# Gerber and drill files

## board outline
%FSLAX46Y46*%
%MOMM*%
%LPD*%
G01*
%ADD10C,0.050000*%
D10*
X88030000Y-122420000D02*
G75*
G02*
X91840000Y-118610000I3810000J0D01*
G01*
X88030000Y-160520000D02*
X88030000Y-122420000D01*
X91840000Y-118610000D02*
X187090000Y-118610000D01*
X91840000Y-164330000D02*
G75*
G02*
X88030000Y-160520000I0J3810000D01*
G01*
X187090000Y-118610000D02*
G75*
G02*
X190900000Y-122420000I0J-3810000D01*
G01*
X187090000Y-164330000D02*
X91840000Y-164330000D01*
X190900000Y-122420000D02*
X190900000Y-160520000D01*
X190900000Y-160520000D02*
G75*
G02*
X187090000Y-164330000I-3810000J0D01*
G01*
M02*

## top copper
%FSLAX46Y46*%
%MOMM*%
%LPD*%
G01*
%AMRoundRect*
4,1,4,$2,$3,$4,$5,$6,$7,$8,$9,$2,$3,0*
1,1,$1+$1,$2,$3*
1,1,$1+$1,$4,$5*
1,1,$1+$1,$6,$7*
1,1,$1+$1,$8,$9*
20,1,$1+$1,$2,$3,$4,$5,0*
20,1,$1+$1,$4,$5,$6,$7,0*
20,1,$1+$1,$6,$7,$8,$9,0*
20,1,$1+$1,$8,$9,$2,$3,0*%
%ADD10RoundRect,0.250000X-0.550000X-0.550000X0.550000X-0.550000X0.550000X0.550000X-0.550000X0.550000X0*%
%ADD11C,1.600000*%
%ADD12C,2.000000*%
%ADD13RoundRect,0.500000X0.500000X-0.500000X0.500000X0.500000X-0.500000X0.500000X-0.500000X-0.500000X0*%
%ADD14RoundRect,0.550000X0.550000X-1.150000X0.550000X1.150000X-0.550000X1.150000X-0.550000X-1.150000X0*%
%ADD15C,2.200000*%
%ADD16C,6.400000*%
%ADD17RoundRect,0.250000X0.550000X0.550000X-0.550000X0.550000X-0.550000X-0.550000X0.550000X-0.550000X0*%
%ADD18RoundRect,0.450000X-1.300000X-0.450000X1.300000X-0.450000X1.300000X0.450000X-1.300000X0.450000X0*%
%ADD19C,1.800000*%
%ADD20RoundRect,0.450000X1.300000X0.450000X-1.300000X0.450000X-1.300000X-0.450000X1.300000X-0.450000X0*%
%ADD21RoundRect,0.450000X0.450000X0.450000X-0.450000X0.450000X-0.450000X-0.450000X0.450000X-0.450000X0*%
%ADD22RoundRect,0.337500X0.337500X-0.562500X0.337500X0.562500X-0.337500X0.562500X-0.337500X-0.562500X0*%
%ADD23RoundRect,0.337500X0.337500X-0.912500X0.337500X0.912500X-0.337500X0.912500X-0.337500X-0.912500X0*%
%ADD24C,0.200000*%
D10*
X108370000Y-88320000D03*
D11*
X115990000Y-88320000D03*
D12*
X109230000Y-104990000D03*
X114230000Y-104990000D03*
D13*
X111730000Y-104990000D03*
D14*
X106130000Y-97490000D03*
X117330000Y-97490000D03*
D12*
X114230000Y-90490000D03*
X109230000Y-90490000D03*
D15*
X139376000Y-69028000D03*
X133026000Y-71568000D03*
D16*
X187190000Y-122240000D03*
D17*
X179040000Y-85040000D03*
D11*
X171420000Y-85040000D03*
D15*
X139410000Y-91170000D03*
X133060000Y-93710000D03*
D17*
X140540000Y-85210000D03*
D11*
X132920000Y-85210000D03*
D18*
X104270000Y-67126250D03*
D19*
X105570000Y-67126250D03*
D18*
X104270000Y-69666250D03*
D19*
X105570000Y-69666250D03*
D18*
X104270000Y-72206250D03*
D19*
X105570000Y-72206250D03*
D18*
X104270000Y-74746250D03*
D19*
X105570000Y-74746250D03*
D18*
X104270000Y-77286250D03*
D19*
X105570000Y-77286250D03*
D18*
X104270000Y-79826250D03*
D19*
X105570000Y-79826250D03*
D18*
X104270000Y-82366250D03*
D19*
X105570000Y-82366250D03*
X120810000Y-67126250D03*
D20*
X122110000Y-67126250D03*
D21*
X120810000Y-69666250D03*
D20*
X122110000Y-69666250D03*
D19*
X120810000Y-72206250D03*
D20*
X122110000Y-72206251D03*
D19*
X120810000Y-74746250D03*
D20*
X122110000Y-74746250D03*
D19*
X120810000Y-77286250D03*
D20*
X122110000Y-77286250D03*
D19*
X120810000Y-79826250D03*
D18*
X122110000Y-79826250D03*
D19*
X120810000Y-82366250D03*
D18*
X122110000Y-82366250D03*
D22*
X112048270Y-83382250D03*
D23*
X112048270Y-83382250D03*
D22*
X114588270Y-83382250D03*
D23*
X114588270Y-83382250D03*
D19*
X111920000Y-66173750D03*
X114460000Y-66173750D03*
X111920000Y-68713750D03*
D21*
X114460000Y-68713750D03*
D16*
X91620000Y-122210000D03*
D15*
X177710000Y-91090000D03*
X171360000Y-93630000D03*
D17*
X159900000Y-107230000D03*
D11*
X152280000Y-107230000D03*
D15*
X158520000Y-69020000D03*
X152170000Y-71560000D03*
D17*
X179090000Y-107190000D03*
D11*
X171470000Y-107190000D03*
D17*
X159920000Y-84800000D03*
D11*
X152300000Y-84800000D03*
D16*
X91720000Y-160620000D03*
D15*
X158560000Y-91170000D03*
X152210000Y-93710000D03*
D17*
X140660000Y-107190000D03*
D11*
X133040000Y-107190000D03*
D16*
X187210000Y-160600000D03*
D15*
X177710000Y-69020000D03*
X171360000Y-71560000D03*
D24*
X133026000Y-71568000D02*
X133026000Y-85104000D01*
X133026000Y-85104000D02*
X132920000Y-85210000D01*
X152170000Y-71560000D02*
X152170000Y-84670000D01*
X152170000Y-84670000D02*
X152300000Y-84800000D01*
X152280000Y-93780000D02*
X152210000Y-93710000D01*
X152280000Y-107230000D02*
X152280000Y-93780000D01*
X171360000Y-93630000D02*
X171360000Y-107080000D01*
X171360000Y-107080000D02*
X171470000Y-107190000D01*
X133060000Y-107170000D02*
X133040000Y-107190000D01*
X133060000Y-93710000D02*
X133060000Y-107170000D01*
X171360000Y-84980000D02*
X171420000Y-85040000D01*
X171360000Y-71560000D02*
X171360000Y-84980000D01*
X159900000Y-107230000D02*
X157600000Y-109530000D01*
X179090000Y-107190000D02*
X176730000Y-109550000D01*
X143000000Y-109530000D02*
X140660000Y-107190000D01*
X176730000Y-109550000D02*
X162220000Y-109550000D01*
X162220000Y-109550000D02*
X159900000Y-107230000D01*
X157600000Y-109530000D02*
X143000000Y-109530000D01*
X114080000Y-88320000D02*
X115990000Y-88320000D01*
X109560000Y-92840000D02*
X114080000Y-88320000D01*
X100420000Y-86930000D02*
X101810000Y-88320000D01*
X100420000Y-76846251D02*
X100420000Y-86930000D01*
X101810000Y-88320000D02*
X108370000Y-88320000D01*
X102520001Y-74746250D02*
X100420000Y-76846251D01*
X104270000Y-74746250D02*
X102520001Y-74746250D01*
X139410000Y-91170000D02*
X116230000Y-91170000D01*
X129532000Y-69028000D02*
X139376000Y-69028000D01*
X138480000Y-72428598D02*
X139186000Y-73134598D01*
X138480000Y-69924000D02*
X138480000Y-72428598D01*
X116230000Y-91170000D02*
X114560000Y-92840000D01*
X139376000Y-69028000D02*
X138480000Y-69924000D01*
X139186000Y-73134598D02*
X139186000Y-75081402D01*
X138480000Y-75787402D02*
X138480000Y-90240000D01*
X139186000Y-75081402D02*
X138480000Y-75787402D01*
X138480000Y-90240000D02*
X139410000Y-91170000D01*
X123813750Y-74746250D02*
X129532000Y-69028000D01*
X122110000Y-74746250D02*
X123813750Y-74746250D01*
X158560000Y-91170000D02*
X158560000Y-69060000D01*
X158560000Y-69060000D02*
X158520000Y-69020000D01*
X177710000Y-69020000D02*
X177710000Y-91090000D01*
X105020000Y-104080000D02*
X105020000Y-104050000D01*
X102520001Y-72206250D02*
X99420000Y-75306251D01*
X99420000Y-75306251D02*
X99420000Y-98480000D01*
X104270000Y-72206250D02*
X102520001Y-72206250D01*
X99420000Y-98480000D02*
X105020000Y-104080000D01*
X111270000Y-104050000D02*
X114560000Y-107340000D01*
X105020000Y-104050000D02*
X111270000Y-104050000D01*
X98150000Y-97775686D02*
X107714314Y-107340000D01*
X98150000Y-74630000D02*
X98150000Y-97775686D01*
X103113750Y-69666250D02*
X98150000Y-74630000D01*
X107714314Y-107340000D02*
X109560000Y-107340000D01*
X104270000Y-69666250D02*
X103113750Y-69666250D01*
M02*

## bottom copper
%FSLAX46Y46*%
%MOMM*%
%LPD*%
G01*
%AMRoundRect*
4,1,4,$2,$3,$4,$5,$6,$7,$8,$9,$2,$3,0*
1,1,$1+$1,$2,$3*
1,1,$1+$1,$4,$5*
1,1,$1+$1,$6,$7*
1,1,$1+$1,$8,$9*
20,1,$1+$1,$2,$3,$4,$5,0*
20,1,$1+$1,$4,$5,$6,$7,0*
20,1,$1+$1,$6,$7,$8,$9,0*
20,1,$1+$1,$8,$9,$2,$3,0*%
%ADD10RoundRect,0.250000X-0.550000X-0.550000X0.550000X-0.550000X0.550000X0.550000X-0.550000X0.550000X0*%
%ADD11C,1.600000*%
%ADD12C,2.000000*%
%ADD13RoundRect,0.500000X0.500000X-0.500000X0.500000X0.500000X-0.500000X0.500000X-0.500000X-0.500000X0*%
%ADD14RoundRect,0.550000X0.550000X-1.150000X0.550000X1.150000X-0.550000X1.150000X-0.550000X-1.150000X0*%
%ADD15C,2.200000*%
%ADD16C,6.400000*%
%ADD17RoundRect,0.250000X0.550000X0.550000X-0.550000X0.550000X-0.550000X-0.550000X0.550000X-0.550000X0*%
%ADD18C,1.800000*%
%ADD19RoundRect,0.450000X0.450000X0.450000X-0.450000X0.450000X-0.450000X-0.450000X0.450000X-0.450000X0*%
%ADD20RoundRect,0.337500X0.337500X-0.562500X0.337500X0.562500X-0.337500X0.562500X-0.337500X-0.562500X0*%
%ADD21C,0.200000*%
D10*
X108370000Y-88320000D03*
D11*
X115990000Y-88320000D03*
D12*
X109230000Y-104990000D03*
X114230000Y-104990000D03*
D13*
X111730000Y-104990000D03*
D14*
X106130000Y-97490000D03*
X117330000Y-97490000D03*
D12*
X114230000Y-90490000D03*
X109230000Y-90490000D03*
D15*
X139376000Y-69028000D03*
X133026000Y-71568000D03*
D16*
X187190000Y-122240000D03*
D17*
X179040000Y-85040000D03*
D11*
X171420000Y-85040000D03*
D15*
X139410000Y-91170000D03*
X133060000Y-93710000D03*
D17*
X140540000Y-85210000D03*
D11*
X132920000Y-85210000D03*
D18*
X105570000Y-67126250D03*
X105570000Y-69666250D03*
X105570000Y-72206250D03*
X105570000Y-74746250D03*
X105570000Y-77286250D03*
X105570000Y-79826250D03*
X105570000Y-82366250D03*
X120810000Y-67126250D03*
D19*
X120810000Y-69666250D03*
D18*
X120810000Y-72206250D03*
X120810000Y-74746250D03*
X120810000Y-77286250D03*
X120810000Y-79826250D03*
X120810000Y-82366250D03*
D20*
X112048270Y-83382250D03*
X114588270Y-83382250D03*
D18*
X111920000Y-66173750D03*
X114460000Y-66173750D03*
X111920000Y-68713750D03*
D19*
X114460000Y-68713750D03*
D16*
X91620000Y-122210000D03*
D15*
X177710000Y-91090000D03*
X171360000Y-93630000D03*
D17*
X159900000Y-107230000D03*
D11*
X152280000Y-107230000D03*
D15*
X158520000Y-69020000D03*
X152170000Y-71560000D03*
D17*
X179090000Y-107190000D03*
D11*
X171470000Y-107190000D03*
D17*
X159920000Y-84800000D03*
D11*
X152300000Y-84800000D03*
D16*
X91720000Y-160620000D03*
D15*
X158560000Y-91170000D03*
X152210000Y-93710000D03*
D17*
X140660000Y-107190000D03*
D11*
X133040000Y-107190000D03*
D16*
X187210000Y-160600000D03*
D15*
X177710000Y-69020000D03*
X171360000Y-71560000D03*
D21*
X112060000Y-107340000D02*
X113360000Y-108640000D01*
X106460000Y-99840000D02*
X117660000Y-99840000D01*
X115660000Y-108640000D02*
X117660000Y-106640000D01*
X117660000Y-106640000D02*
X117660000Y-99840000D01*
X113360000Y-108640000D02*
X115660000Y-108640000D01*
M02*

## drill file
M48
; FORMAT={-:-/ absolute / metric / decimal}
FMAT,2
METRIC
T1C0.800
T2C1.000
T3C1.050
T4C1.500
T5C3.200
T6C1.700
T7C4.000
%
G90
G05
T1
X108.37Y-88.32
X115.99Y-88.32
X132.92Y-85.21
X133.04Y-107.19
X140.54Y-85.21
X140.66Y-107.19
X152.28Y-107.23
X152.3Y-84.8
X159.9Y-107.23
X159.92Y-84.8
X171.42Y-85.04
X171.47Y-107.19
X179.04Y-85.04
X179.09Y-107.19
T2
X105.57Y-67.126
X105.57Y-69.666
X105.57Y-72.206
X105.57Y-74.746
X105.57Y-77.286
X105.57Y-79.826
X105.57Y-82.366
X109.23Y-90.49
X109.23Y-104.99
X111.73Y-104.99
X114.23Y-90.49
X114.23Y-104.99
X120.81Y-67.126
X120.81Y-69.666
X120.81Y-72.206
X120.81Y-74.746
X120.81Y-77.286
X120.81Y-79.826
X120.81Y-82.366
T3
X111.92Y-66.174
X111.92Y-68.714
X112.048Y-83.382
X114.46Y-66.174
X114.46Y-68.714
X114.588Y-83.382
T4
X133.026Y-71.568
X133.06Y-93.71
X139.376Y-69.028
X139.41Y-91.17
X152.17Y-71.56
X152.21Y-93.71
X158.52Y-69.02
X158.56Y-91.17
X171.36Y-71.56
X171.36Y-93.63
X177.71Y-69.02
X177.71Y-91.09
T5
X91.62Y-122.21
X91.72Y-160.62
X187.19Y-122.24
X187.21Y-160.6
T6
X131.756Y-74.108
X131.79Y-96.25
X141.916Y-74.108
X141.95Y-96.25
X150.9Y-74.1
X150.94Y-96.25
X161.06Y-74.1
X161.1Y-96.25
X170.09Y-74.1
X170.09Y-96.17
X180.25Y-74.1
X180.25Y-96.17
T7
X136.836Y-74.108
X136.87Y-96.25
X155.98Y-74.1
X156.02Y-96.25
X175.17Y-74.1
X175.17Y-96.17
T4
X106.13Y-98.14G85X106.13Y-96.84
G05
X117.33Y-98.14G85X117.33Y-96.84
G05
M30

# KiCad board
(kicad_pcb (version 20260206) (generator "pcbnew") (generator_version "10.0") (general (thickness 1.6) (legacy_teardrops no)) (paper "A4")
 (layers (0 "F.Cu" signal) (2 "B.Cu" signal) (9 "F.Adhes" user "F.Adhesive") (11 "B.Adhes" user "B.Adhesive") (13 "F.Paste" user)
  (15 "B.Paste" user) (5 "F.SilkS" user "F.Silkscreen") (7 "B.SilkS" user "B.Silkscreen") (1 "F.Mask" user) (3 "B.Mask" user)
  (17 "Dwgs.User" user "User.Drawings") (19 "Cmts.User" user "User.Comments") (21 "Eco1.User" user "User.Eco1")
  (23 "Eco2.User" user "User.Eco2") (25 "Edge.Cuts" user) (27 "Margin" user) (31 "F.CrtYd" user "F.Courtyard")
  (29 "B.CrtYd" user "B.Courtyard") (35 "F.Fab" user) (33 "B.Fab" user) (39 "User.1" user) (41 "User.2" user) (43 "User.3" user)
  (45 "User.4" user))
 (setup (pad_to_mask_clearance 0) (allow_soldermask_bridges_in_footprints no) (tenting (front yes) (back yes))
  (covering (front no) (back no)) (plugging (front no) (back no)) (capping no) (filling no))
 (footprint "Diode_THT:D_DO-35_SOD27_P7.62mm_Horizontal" (layer "F.Cu") (at 108.37 88.32)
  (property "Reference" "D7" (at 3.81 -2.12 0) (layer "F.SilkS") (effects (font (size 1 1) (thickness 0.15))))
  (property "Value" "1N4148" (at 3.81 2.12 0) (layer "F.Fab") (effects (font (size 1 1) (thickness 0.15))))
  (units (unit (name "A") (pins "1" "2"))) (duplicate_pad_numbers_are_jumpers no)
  (pad "1" thru_hole roundrect (at 0 0) (size 1.6 1.6) (drill 0.8) (layers "*.Cu" "*.Mask") (remove_unused_layers no)
   (roundrect_rratio 0.15625) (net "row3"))
  (pad "2" thru_hole circle (at 7.62 0) (size 1.6 1.6) (drill 0.8) (layers "*.Cu" "*.Mask") (remove_unused_layers no) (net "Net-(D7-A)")))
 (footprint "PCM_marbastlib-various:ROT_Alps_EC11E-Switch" (layer "F.Cu") (at 111.73 97.49)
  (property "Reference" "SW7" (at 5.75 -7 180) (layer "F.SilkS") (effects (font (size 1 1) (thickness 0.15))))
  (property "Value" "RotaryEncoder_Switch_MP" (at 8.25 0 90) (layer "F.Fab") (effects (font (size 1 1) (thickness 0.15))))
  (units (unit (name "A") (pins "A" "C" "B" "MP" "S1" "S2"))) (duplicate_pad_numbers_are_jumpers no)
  (pad "A" thru_hole circle (at -2.5 7.5 90) (size 2 2) (drill 1) (layers "*.Cu" "B.Mask") (remove_unused_layers no) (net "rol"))
  (pad "B" thru_hole circle (at 2.5 7.5 90) (size 2 2) (drill 1) (layers "*.Cu" "B.Mask") (remove_unused_layers no) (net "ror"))
  (pad "C" thru_hole roundrect (at 0 7.5 90) (size 2 2) (drill 1) (layers "*.Cu" "B.Mask") (remove_unused_layers no) (roundrect_rratio 0.25)
   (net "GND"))
  (pad "MP" thru_hole roundrect (at -5.6 0 90) (size 3.4 2.2) (drill oval 2.8 1.5) (layers "*.Cu" "B.Mask") (remove_unused_layers no)
   (roundrect_rratio 0.25) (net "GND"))
  (pad "MP" thru_hole roundrect (at 5.6 0 90) (size 3.4 2.2) (drill oval 2.8 1.5) (layers "*.Cu" "B.Mask") (remove_unused_layers no)
   (roundrect_rratio 0.25) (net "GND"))
  (pad "S1" thru_hole circle (at 2.5 -7 90) (size 2 2) (drill 1) (layers "*.Cu" "B.Mask") (remove_unused_layers no) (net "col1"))
  (pad "S2" thru_hole circle (at -2.5 -7 90) (size 2 2) (drill 1) (layers "*.Cu" "B.Mask") (remove_unused_layers no) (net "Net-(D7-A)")))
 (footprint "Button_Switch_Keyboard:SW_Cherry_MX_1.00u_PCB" (layer "F.Cu") (at 139.376 69.028)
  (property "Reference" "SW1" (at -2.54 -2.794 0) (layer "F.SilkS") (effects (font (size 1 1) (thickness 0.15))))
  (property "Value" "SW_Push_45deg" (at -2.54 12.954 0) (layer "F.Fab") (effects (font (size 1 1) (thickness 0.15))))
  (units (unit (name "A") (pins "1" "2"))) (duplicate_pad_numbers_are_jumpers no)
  (pad "" np_thru_hole circle (at -7.62 5.08) (size 1.7 1.7) (drill 1.7) (layers "*.Cu" "*.Mask"))
  (pad "" np_thru_hole circle (at -2.54 5.08) (size 4 4) (drill 4) (layers "*.Cu" "*.Mask"))
  (pad "" np_thru_hole circle (at 2.54 5.08) (size 1.7 1.7) (drill 1.7) (layers "*.Cu" "*.Mask"))
  (pad "1" thru_hole circle (at 0 0) (size 2.2 2.2) (drill 1.5) (layers "*.Cu" "*.Mask") (remove_unused_layers no) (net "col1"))
  (pad "2" thru_hole circle (at -6.35 2.54) (size 2.2 2.2) (drill 1.5) (layers "*.Cu" "*.Mask") (remove_unused_layers no) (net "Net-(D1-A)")))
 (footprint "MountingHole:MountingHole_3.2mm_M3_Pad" (layer "F.Cu") (at 187.19 122.24)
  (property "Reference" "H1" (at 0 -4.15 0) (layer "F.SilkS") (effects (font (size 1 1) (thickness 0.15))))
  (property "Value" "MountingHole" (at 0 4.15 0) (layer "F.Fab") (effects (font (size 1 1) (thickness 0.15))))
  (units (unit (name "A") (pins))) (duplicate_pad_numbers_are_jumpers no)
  (pad "1" thru_hole circle (at 0 0) (size 6.4 6.4) (drill 3.2) (layers "*.Cu" "*.Mask") (remove_unused_layers no) (zone_connect 2)))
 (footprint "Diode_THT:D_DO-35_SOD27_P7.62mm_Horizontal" (layer "F.Cu") (at 179.04 85.04 180)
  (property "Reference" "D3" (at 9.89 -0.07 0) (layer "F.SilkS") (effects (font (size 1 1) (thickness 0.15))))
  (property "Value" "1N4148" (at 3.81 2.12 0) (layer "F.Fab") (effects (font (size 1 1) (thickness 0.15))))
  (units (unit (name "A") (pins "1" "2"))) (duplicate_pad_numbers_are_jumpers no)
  (pad "1" thru_hole roundrect (at 0 0 180) (size 1.6 1.6) (drill 0.8) (layers "*.Cu" "*.Mask") (remove_unused_layers no)
   (roundrect_rratio 0.15625) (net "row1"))
  (pad "2" thru_hole circle (at 7.62 0 180) (size 1.6 1.6) (drill 0.8) (layers "*.Cu" "*.Mask") (remove_unused_layers no) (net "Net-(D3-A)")))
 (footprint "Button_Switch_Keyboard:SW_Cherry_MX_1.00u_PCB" (layer "F.Cu") (at 139.41 91.17)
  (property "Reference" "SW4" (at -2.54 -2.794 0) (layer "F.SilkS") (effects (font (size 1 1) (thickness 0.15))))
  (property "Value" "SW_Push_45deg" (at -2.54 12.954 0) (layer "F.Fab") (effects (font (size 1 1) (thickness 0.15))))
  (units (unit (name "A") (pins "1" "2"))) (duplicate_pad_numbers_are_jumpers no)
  (pad "" np_thru_hole circle (at -7.62 5.08) (size 1.7 1.7) (drill 1.7) (layers "*.Cu" "*.Mask"))
  (pad "" np_thru_hole circle (at -2.54 5.08) (size 4 4) (drill 4) (layers "*.Cu" "*.Mask"))
  (pad "" np_thru_hole circle (at 2.54 5.08) (size 1.7 1.7) (drill 1.7) (layers "*.Cu" "*.Mask"))
  (pad "1" thru_hole circle (at 0 0) (size 2.2 2.2) (drill 1.5) (layers "*.Cu" "*.Mask") (remove_unused_layers no) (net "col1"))
  (pad "2" thru_hole circle (at -6.35 2.54) (size 2.2 2.2) (drill 1.5) (layers "*.Cu" "*.Mask") (remove_unused_layers no) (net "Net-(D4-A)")))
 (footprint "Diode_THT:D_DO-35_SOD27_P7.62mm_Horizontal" (layer "F.Cu") (at 140.54 85.21 180)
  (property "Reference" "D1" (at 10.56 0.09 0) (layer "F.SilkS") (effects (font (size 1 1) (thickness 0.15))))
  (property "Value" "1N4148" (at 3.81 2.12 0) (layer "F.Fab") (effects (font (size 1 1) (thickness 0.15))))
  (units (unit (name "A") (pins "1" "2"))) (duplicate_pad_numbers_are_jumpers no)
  (pad "1" thru_hole roundrect (at 0 0 180) (size 1.6 1.6) (drill 0.8) (layers "*.Cu" "*.Mask") (remove_unused_layers no)
   (roundrect_rratio 0.15625) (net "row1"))
  (pad "2" thru_hole circle (at 7.62 0 180) (size 1.6 1.6) (drill 0.8) (layers "*.Cu" "*.Mask") (remove_unused_layers no) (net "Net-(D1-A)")))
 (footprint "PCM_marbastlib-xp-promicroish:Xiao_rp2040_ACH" (layer "F.Cu") (at 113.19 74.74625)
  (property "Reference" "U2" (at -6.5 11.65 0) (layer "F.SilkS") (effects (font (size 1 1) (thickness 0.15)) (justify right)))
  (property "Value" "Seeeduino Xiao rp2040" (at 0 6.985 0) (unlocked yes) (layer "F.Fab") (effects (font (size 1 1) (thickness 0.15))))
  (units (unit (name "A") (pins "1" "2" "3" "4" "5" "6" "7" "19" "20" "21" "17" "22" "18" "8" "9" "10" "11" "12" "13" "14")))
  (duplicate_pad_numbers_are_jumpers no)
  (pad "1" smd roundrect (at -8.92 -7.62) (size 3.5 1.8) (layers "F.Cu" "F.Mask") (roundrect_rratio 0.25) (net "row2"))
  (pad "1" thru_hole circle (at -7.62 -7.62) (size 1.8 1.8) (drill 1) (layers "*.Cu" "*.Mask") (remove_unused_layers no) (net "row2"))
  (pad "2" smd roundrect (at -8.92 -5.08) (size 3.5 1.8) (layers "F.Cu" "F.Mask") (roundrect_rratio 0.25) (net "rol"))
  (pad "2" thru_hole circle (at -7.62 -5.08) (size 1.8 1.8) (drill 1) (layers "*.Cu" "*.Mask") (remove_unused_layers no) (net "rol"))
  (pad "3" smd roundrect (at -8.92 -2.54) (size 3.5 1.8) (layers "F.Cu" "F.Mask") (roundrect_rratio 0.25) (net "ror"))
  (pad "3" thru_hole circle (at -7.62 -2.54) (size 1.8 1.8) (drill 1) (layers "*.Cu" "*.Mask") (remove_unused_layers no) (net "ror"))
  (pad "4" smd roundrect (at -8.92 0) (size 3.5 1.8) (layers "F.Cu" "F.Mask") (roundrect_rratio 0.25) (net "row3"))
  (pad "4" thru_hole circle (at -7.62 0) (size 1.8 1.8) (drill 1) (layers "*.Cu" "*.Mask") (remove_unused_layers no) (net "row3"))
  (pad "5" smd roundrect (at -8.92 2.54) (size 3.5 1.8) (layers "F.Cu" "F.Mask") (roundrect_rratio 0.25) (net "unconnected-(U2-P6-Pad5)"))
  (pad "5" thru_hole circle (at -7.62 2.54) (size 1.8 1.8) (drill 1) (layers "*.Cu" "*.Mask") (remove_unused_layers no)
   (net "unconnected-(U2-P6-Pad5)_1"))
  (pad "6" smd roundrect (at -8.92 5.08) (size 3.5 1.8) (layers "F.Cu" "F.Mask") (roundrect_rratio 0.25) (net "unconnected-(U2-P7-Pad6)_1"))
  (pad "6" thru_hole circle (at -7.62 5.08) (size 1.8 1.8) (drill 1) (layers "*.Cu" "*.Mask") (remove_unused_layers no)
   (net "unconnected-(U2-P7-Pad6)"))
  (pad "7" smd roundrect (at -8.92 7.62) (size 3.5 1.8) (layers "F.Cu" "F.Mask") (roundrect_rratio 0.25) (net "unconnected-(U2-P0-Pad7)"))
  (pad "7" thru_hole circle (at -7.62 7.62) (size 1.8 1.8) (drill 1) (layers "*.Cu" "*.Mask") (remove_unused_layers no)
   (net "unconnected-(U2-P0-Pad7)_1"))
  (pad "8" thru_hole circle (at 7.62 -7.62 180) (size 1.8 1.8) (drill 1) (layers "*.Cu" "*.Mask") (remove_unused_layers no) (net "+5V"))
  (pad "8" smd roundrect (at 8.92 -7.62 180) (size 3.5 1.8) (layers "F.Cu" "F.Mask") (roundrect_rratio 0.25) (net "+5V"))
  (pad "9" thru_hole roundrect (at 7.62 -5.08 180) (size 1.8 1.8) (drill 1) (layers "*.Cu" "*.Mask") (remove_unused_layers no)
   (roundrect_rratio 0.25) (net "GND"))
  (pad "9" smd roundrect (at 8.92 -5.08 180) (size 3.5 1.8) (layers "F.Cu" "F.Mask") (roundrect_rratio 0.25) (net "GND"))
  (pad "10" thru_hole circle (at 7.62 -2.54 180) (size 1.8 1.8) (drill 1) (layers "*.Cu" "*.Mask") (remove_unused_layers no) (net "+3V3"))
  (pad "10" smd roundrect (at 8.92 -2.539999 180) (size 3.5 1.8) (layers "F.Cu" "F.Mask") (roundrect_rratio 0.25) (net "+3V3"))
  (pad "11" thru_hole circle (at 7.62 0 180) (size 1.8 1.8) (drill 1) (layers "*.Cu" "*.Mask") (remove_unused_layers no) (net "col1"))
  (pad "11" smd roundrect (at 8.92 0 180) (size 3.5 1.8) (layers "F.Cu" "F.Mask") (roundrect_rratio 0.25) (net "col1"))
  (pad "12" thru_hole circle (at 7.62 2.54 180) (size 1.8 1.8) (drill 1) (layers "*.Cu" "*.Mask") (remove_unused_layers no) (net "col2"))
  (pad "12" smd roundrect (at 8.92 2.54 180) (size 3.5 1.8) (layers "F.Cu" "F.Mask") (roundrect_rratio 0.25) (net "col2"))
  (pad "13" thru_hole circle (at 7.62 5.08) (size 1.8 1.8) (drill 1) (layers "*.Cu" "*.Mask") (remove_unused_layers no) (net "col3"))
  (pad "13" smd roundrect (at 8.92 5.08) (size 3.5 1.8) (layers "F.Cu" "F.Mask") (roundrect_rratio 0.25) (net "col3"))
  (pad "14" thru_hole circle (at 7.62 7.62) (size 1.8 1.8) (drill 1) (layers "*.Cu" "*.Mask") (remove_unused_layers no) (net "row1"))
  (pad "14" smd roundrect (at 8.92 7.62) (size 3.5 1.8) (layers "F.Cu" "F.Mask") (roundrect_rratio 0.25) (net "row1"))
  (pad "17" thru_hole roundrect (at -1.14173 8.636 90) (size 1.8 1.35) (drill 1.05) (layers "*.Cu" "*.Mask") (remove_unused_layers no)
   (roundrect_rratio 0.25) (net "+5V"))
  (pad "17" smd roundrect (at -1.14173 8.636 90) (size 2.5 1.35) (layers "F.Cu" "F.Mask") (roundrect_rratio 0.25) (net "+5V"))
  (pad "18" thru_hole roundrect (at 1.39827 8.636 90) (size 1.8 1.35) (drill 1.05) (layers "*.Cu" "*.Mask") (remove_unused_layers no)
   (roundrect_rratio 0.25) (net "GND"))
  (pad "18" smd roundrect (at 1.39827 8.636 90) (size 2.5 1.35) (layers "F.Cu" "F.Mask") (roundrect_rratio 0.25) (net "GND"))
  (pad "19" thru_hole circle (at -1.27 -8.5725 180) (size 1.8 1.8) (drill 1.05) (layers "*.Cu" "*.Mask") (remove_unused_layers no)
   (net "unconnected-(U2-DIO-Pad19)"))
  (pad "20" thru_hole circle (at 1.27 -8.5725 180) (size 1.8 1.8) (drill 1.05) (layers "*.Cu" "*.Mask") (remove_unused_layers no)
   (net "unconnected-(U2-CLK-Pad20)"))
  (pad "21" thru_hole circle (at -1.27 -6.0325 180) (size 1.8 1.8) (drill 1.05) (layers "*.Cu" "*.Mask") (remove_unused_layers no)
   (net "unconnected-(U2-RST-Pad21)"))
  (pad "22" thru_hole roundrect (at 1.27 -6.0325 180) (size 1.8 1.8) (drill 1.05) (layers "*.Cu" "*.Mask") (remove_unused_layers no)
   (roundrect_rratio 0.25) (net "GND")))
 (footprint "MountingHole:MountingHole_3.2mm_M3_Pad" (layer "F.Cu") (at 91.62 122.21)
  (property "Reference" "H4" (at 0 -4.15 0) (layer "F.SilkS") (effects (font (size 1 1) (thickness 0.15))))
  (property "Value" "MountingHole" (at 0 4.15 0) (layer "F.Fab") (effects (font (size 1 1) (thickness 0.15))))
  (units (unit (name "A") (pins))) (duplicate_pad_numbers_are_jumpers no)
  (pad "1" thru_hole circle (at 0 0) (size 6.4 6.4) (drill 3.2) (layers "*.Cu" "*.Mask") (remove_unused_layers no) (zone_connect 2)))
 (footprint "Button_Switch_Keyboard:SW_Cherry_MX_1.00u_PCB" (layer "F.Cu") (at 177.71 91.09)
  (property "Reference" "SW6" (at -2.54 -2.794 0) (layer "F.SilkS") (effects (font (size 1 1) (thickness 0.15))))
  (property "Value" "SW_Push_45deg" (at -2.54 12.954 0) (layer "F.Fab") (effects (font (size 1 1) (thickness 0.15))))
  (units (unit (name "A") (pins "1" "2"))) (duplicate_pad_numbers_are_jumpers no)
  (pad "" np_thru_hole circle (at -7.62 5.08) (size 1.7 1.7) (drill 1.7) (layers "*.Cu" "*.Mask"))
  (pad "" np_thru_hole circle (at -2.54 5.08) (size 4 4) (drill 4) (layers "*.Cu" "*.Mask"))
  (pad "" np_thru_hole circle (at 2.54 5.08) (size 1.7 1.7) (drill 1.7) (layers "*.Cu" "*.Mask"))
  (pad "1" thru_hole circle (at 0 0) (size 2.2 2.2) (drill 1.5) (layers "*.Cu" "*.Mask") (remove_unused_layers no) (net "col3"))
  (pad "2" thru_hole circle (at -6.35 2.54) (size 2.2 2.2) (drill 1.5) (layers "*.Cu" "*.Mask") (remove_unused_layers no) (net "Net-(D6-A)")))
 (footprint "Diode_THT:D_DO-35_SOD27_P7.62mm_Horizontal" (layer "F.Cu") (at 159.9 107.23 180)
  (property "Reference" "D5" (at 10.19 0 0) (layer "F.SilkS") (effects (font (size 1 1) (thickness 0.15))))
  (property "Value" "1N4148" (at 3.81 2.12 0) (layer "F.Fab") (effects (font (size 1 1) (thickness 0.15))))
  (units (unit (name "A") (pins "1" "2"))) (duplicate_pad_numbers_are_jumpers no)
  (pad "1" thru_hole roundrect (at 0 0 180) (size 1.6 1.6) (drill 0.8) (layers "*.Cu" "*.Mask") (remove_unused_layers no)
   (roundrect_rratio 0.15625) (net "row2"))
  (pad "2" thru_hole circle (at 7.62 0 180) (size 1.6 1.6) (drill 0.8) (layers "*.Cu" "*.Mask") (remove_unused_layers no) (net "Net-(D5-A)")))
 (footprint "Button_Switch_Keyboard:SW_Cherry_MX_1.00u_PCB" (layer "F.Cu") (at 158.52 69.02)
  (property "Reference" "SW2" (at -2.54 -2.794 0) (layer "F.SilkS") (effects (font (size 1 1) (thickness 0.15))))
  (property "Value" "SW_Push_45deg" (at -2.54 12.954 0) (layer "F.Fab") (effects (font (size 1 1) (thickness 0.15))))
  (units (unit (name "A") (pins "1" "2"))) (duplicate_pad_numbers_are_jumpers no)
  (pad "" np_thru_hole circle (at -7.62 5.08) (size 1.7 1.7) (drill 1.7) (layers "*.Cu" "*.Mask"))
  (pad "" np_thru_hole circle (at -2.54 5.08) (size 4 4) (drill 4) (layers "*.Cu" "*.Mask"))
  (pad "" np_thru_hole circle (at 2.54 5.08) (size 1.7 1.7) (drill 1.7) (layers "*.Cu" "*.Mask"))
  (pad "1" thru_hole circle (at 0 0) (size 2.2 2.2) (drill 1.5) (layers "*.Cu" "*.Mask") (remove_unused_layers no) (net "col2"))
  (pad "2" thru_hole circle (at -6.35 2.54) (size 2.2 2.2) (drill 1.5) (layers "*.Cu" "*.Mask") (remove_unused_layers no) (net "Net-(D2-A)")))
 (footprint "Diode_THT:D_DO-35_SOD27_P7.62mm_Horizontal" (layer "F.Cu") (at 179.09 107.19 180)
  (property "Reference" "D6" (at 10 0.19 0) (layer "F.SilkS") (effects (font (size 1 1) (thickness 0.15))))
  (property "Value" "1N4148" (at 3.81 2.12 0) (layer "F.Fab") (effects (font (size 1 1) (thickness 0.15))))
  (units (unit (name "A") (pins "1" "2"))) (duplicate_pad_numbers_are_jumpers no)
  (pad "1" thru_hole roundrect (at 0 0 180) (size 1.6 1.6) (drill 0.8) (layers "*.Cu" "*.Mask") (remove_unused_layers no)
   (roundrect_rratio 0.15625) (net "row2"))
  (pad "2" thru_hole circle (at 7.62 0 180) (size 1.6 1.6) (drill 0.8) (layers "*.Cu" "*.Mask") (remove_unused_layers no) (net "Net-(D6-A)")))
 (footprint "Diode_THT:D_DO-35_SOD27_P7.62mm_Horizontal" (layer "F.Cu") (at 159.92 84.8 180)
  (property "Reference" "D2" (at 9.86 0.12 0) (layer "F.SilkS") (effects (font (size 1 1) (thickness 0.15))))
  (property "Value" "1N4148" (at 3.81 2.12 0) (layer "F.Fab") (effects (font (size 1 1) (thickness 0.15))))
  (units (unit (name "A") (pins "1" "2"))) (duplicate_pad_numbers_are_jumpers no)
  (pad "1" thru_hole roundrect (at 0 0 180) (size 1.6 1.6) (drill 0.8) (layers "*.Cu" "*.Mask") (remove_unused_layers no)
   (roundrect_rratio 0.15625) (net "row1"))
  (pad "2" thru_hole circle (at 7.62 0 180) (size 1.6 1.6) (drill 0.8) (layers "*.Cu" "*.Mask") (remove_unused_layers no) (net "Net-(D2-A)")))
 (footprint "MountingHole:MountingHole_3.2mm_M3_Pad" (layer "F.Cu") (at 91.72 160.62)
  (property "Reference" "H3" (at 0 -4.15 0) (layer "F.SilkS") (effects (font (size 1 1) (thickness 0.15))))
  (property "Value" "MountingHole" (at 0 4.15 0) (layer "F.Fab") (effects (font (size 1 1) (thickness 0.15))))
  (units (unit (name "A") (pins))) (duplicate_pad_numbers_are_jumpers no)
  (pad "1" thru_hole circle (at 0 0) (size 6.4 6.4) (drill 3.2) (layers "*.Cu" "*.Mask") (remove_unused_layers no) (zone_connect 2)))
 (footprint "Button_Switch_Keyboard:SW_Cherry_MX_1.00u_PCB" (layer "F.Cu") (at 158.56 91.17)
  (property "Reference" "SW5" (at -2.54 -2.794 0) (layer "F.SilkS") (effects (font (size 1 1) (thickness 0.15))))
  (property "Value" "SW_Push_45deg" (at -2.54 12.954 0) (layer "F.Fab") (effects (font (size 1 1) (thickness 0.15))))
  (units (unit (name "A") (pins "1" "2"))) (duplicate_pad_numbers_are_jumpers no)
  (pad "" np_thru_hole circle (at -7.62 5.08) (size 1.7 1.7) (drill 1.7) (layers "*.Cu" "*.Mask"))
  (pad "" np_thru_hole circle (at -2.54 5.08) (size 4 4) (drill 4) (layers "*.Cu" "*.Mask"))
  (pad "" np_thru_hole circle (at 2.54 5.08) (size 1.7 1.7) (drill 1.7) (layers "*.Cu" "*.Mask"))
  (pad "1" thru_hole circle (at 0 0) (size 2.2 2.2) (drill 1.5) (layers "*.Cu" "*.Mask") (remove_unused_layers no) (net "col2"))
  (pad "2" thru_hole circle (at -6.35 2.54) (size 2.2 2.2) (drill 1.5) (layers "*.Cu" "*.Mask") (remove_unused_layers no) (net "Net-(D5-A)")))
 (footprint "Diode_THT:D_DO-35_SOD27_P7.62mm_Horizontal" (layer "F.Cu") (at 140.66 107.19 180)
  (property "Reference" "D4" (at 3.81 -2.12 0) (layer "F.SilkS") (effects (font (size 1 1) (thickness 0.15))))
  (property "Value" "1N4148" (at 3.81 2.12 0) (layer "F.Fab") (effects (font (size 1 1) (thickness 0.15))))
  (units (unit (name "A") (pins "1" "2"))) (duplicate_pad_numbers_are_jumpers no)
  (pad "1" thru_hole roundrect (at 0 0 180) (size 1.6 1.6) (drill 0.8) (layers "*.Cu" "*.Mask") (remove_unused_layers no)
   (roundrect_rratio 0.15625) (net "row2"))
  (pad "2" thru_hole circle (at 7.62 0 180) (size 1.6 1.6) (drill 0.8) (layers "*.Cu" "*.Mask") (remove_unused_layers no) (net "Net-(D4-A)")))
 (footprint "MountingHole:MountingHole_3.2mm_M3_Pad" (layer "F.Cu") (at 187.21 160.6)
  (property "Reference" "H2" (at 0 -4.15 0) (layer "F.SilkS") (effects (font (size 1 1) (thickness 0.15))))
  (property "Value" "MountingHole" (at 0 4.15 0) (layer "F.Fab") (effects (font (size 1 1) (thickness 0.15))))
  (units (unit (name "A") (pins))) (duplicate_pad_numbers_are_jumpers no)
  (pad "1" thru_hole circle (at 0 0) (size 6.4 6.4) (drill 3.2) (layers "*.Cu" "*.Mask") (remove_unused_layers no) (zone_connect 2)))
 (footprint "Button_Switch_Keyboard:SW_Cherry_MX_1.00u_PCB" (layer "F.Cu") (at 177.71 69.02)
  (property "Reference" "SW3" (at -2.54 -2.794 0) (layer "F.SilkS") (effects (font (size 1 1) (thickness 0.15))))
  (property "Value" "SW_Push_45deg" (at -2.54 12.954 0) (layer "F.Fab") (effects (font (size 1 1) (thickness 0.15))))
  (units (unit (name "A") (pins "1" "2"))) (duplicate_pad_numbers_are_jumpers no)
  (pad "" np_thru_hole circle (at -7.62 5.08) (size 1.7 1.7) (drill 1.7) (layers "*.Cu" "*.Mask"))
  (pad "" np_thru_hole circle (at -2.54 5.08) (size 4 4) (drill 4) (layers "*.Cu" "*.Mask"))
  (pad "" np_thru_hole circle (at 2.54 5.08) (size 1.7 1.7) (drill 1.7) (layers "*.Cu" "*.Mask"))
  (pad "1" thru_hole circle (at 0 0) (size 2.2 2.2) (drill 1.5) (layers "*.Cu" "*.Mask") (remove_unused_layers no) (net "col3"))
  (pad "2" thru_hole circle (at -6.35 2.54) (size 2.2 2.2) (drill 1.5) (layers "*.Cu" "*.Mask") (remove_unused_layers no) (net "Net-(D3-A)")))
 (gr_arc (start 88.03 122.42) (mid 89.145923 119.725923) (end 91.84 118.61) (stroke (width 0.05) (type default)) (layer "Edge.Cuts"))
 (gr_line (start 88.03 160.52) (end 88.03 122.42) (stroke (width 0.05) (type default)) (layer "Edge.Cuts"))
 (gr_line (start 91.84 118.61) (end 187.09 118.61) (stroke (width 0.05) (type default)) (layer "Edge.Cuts"))
 (gr_arc (start 91.84 164.33) (mid 89.145923 163.214077) (end 88.03 160.52) (stroke (width 0.05) (type default)) (layer "Edge.Cuts"))
 (gr_arc (start 187.09 118.61) (mid 189.784077 119.725923) (end 190.9 122.42) (stroke (width 0.05) (type default)) (layer "Edge.Cuts"))
 (gr_line (start 187.09 164.33) (end 91.84 164.33) (stroke (width 0.05) (type default)) (layer "Edge.Cuts"))
 (gr_line (start 190.9 122.42) (end 190.9 160.52) (stroke (width 0.05) (type default)) (layer "Edge.Cuts"))
 (gr_arc (start 190.9 160.52) (mid 189.784077 163.214077) (end 187.09 164.33) (stroke (width 0.05) (type default)) (layer "Edge.Cuts"))
 (segment (start 133.026 71.568) (end 133.026 85.104) (width 0.2) (layer "F.Cu") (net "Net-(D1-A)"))
 (segment (start 133.026 85.104) (end 132.92 85.21) (width 0.2) (layer "F.Cu") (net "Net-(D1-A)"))
 (segment (start 152.17 71.56) (end 152.17 84.67) (width 0.2) (layer "F.Cu") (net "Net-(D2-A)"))
 (segment (start 152.17 84.67) (end 152.3 84.8) (width 0.2) (layer "F.Cu") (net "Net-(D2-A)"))
 (segment (start 152.28 93.78) (end 152.21 93.71) (width 0.2) (layer "F.Cu") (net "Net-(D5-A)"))
 (segment (start 152.28 107.23) (end 152.28 93.78) (width 0.2) (layer "F.Cu") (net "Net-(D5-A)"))
 (segment (start 171.36 93.63) (end 171.36 107.08) (width 0.2) (layer "F.Cu") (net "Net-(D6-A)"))
 (segment (start 171.36 107.08) (end 171.47 107.19) (width 0.2) (layer "F.Cu") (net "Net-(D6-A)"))
 (segment (start 133.06 107.17) (end 133.04 107.19) (width 0.2) (layer "F.Cu") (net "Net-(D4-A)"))
 (segment (start 133.06 93.71) (end 133.06 107.17) (width 0.2) (layer "F.Cu") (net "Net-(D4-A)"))
 (segment (start 171.36 84.98) (end 171.42 85.04) (width 0.2) (layer "F.Cu") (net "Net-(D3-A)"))
 (segment (start 171.36 71.56) (end 171.36 84.98) (width 0.2) (layer "F.Cu") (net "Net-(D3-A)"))
 (segment (start 159.9 107.23) (end 157.6 109.53) (width 0.2) (layer "F.Cu") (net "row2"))
 (segment (start 179.09 107.19) (end 176.73 109.55) (width 0.2) (layer "F.Cu") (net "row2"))
 (segment (start 143 109.53) (end 140.66 107.19) (width 0.2) (layer "F.Cu") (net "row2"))
 (segment (start 176.73 109.55) (end 162.22 109.55) (width 0.2) (layer "F.Cu") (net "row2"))
 (segment (start 162.22 109.55) (end 159.9 107.23) (width 0.2) (layer "F.Cu") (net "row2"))
 (segment (start 157.6 109.53) (end 143 109.53) (width 0.2) (layer "F.Cu") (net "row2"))
 (segment (start 114.08 88.32) (end 115.99 88.32) (width 0.2) (layer "F.Cu") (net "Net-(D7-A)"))
 (segment (start 109.56 92.84) (end 114.08 88.32) (width 0.2) (layer "F.Cu") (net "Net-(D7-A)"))
 (segment (start 100.42 86.93) (end 101.81 88.32) (width 0.2) (layer "F.Cu") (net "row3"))
 (segment (start 100.42 76.846251) (end 100.42 86.93) (width 0.2) (layer "F.Cu") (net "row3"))
 (segment (start 101.81 88.32) (end 108.37 88.32) (width 0.2) (layer "F.Cu") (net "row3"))
 (segment (start 102.520001 74.74625) (end 100.42 76.846251) (width 0.2) (layer "F.Cu") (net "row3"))
 (segment (start 104.27 74.74625) (end 102.520001 74.74625) (width 0.2) (layer "F.Cu") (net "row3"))
 (segment (start 139.41 91.17) (end 116.23 91.17) (width 0.2) (layer "F.Cu") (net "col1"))
 (segment (start 129.532 69.028) (end 139.376 69.028) (width 0.2) (layer "F.Cu") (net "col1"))
 (segment (start 138.48 72.428598) (end 139.186 73.134598) (width 0.2) (layer "F.Cu") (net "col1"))
 (segment (start 138.48 69.924) (end 138.48 72.428598) (width 0.2) (layer "F.Cu") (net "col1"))
 (segment (start 116.23 91.17) (end 114.56 92.84) (width 0.2) (layer "F.Cu") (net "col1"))
 (segment (start 139.376 69.028) (end 138.48 69.924) (width 0.2) (layer "F.Cu") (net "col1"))
 (segment (start 139.186 73.134598) (end 139.186 75.081402) (width 0.2) (layer "F.Cu") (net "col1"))
 (segment (start 138.48 75.787402) (end 138.48 90.24) (width 0.2) (layer "F.Cu") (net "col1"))
 (segment (start 139.186 75.081402) (end 138.48 75.787402) (width 0.2) (layer "F.Cu") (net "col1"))
 (segment (start 138.48 90.24) (end 139.41 91.17) (width 0.2) (layer "F.Cu") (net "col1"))
 (segment (start 123.81375 74.74625) (end 129.532 69.028) (width 0.2) (layer "F.Cu") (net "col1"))
 (segment (start 122.11 74.74625) (end 123.81375 74.74625) (width 0.2) (layer "F.Cu") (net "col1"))
 (segment (start 158.56 91.17) (end 158.56 69.06) (width 0.2) (layer "F.Cu") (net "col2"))
 (segment (start 158.56 69.06) (end 158.52 69.02) (width 0.2) (layer "F.Cu") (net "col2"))
 (segment (start 177.71 69.02) (end 177.71 91.09) (width 0.2) (layer "F.Cu") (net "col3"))
 (segment (start 112.06 107.34) (end 113.36 108.64) (width 0.2) (layer "B.Cu") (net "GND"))
 (segment (start 106.46 99.84) (end 117.66 99.84) (width 0.2) (layer "B.Cu") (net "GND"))
 (segment (start 115.66 108.64) (end 117.66 106.64) (width 0.2) (layer "B.Cu") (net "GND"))
 (segment (start 117.66 106.64) (end 117.66 99.84) (width 0.2) (layer "B.Cu") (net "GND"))
 (segment (start 113.36 108.64) (end 115.66 108.64) (width 0.2) (layer "B.Cu") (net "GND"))
 (segment (start 105.02 104.08) (end 105.02 104.05) (width 0.2) (layer "F.Cu") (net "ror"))
 (segment (start 102.520001 72.20625) (end 99.42 75.306251) (width 0.2) (layer "F.Cu") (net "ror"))
 (segment (start 99.42 75.306251) (end 99.42 98.48) (width 0.2) (layer "F.Cu") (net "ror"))
 (segment (start 104.27 72.20625) (end 102.520001 72.20625) (width 0.2) (layer "F.Cu") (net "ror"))
 (segment (start 99.42 98.48) (end 105.02 104.08) (width 0.2) (layer "F.Cu") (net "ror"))
 (segment (start 111.27 104.05) (end 114.56 107.34) (width 0.2) (layer "F.Cu") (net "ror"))
 (segment (start 105.02 104.05) (end 111.27 104.05) (width 0.2) (layer "F.Cu") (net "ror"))
 (segment (start 98.15 97.775686) (end 107.714314 107.34) (width 0.2) (layer "F.Cu") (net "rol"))
 (segment (start 98.15 74.63) (end 98.15 97.775686) (width 0.2) (layer "F.Cu") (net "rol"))
 (segment (start 103.11375 69.66625) (end 98.15 74.63) (width 0.2) (layer "F.Cu") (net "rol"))
 (segment (start 107.714314 107.34) (end 109.56 107.34) (width 0.2) (layer "F.Cu") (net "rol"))
 (segment (start 104.27 69.66625) (end 103.11375 69.66625) (width 0.2) (layer "F.Cu") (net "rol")))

